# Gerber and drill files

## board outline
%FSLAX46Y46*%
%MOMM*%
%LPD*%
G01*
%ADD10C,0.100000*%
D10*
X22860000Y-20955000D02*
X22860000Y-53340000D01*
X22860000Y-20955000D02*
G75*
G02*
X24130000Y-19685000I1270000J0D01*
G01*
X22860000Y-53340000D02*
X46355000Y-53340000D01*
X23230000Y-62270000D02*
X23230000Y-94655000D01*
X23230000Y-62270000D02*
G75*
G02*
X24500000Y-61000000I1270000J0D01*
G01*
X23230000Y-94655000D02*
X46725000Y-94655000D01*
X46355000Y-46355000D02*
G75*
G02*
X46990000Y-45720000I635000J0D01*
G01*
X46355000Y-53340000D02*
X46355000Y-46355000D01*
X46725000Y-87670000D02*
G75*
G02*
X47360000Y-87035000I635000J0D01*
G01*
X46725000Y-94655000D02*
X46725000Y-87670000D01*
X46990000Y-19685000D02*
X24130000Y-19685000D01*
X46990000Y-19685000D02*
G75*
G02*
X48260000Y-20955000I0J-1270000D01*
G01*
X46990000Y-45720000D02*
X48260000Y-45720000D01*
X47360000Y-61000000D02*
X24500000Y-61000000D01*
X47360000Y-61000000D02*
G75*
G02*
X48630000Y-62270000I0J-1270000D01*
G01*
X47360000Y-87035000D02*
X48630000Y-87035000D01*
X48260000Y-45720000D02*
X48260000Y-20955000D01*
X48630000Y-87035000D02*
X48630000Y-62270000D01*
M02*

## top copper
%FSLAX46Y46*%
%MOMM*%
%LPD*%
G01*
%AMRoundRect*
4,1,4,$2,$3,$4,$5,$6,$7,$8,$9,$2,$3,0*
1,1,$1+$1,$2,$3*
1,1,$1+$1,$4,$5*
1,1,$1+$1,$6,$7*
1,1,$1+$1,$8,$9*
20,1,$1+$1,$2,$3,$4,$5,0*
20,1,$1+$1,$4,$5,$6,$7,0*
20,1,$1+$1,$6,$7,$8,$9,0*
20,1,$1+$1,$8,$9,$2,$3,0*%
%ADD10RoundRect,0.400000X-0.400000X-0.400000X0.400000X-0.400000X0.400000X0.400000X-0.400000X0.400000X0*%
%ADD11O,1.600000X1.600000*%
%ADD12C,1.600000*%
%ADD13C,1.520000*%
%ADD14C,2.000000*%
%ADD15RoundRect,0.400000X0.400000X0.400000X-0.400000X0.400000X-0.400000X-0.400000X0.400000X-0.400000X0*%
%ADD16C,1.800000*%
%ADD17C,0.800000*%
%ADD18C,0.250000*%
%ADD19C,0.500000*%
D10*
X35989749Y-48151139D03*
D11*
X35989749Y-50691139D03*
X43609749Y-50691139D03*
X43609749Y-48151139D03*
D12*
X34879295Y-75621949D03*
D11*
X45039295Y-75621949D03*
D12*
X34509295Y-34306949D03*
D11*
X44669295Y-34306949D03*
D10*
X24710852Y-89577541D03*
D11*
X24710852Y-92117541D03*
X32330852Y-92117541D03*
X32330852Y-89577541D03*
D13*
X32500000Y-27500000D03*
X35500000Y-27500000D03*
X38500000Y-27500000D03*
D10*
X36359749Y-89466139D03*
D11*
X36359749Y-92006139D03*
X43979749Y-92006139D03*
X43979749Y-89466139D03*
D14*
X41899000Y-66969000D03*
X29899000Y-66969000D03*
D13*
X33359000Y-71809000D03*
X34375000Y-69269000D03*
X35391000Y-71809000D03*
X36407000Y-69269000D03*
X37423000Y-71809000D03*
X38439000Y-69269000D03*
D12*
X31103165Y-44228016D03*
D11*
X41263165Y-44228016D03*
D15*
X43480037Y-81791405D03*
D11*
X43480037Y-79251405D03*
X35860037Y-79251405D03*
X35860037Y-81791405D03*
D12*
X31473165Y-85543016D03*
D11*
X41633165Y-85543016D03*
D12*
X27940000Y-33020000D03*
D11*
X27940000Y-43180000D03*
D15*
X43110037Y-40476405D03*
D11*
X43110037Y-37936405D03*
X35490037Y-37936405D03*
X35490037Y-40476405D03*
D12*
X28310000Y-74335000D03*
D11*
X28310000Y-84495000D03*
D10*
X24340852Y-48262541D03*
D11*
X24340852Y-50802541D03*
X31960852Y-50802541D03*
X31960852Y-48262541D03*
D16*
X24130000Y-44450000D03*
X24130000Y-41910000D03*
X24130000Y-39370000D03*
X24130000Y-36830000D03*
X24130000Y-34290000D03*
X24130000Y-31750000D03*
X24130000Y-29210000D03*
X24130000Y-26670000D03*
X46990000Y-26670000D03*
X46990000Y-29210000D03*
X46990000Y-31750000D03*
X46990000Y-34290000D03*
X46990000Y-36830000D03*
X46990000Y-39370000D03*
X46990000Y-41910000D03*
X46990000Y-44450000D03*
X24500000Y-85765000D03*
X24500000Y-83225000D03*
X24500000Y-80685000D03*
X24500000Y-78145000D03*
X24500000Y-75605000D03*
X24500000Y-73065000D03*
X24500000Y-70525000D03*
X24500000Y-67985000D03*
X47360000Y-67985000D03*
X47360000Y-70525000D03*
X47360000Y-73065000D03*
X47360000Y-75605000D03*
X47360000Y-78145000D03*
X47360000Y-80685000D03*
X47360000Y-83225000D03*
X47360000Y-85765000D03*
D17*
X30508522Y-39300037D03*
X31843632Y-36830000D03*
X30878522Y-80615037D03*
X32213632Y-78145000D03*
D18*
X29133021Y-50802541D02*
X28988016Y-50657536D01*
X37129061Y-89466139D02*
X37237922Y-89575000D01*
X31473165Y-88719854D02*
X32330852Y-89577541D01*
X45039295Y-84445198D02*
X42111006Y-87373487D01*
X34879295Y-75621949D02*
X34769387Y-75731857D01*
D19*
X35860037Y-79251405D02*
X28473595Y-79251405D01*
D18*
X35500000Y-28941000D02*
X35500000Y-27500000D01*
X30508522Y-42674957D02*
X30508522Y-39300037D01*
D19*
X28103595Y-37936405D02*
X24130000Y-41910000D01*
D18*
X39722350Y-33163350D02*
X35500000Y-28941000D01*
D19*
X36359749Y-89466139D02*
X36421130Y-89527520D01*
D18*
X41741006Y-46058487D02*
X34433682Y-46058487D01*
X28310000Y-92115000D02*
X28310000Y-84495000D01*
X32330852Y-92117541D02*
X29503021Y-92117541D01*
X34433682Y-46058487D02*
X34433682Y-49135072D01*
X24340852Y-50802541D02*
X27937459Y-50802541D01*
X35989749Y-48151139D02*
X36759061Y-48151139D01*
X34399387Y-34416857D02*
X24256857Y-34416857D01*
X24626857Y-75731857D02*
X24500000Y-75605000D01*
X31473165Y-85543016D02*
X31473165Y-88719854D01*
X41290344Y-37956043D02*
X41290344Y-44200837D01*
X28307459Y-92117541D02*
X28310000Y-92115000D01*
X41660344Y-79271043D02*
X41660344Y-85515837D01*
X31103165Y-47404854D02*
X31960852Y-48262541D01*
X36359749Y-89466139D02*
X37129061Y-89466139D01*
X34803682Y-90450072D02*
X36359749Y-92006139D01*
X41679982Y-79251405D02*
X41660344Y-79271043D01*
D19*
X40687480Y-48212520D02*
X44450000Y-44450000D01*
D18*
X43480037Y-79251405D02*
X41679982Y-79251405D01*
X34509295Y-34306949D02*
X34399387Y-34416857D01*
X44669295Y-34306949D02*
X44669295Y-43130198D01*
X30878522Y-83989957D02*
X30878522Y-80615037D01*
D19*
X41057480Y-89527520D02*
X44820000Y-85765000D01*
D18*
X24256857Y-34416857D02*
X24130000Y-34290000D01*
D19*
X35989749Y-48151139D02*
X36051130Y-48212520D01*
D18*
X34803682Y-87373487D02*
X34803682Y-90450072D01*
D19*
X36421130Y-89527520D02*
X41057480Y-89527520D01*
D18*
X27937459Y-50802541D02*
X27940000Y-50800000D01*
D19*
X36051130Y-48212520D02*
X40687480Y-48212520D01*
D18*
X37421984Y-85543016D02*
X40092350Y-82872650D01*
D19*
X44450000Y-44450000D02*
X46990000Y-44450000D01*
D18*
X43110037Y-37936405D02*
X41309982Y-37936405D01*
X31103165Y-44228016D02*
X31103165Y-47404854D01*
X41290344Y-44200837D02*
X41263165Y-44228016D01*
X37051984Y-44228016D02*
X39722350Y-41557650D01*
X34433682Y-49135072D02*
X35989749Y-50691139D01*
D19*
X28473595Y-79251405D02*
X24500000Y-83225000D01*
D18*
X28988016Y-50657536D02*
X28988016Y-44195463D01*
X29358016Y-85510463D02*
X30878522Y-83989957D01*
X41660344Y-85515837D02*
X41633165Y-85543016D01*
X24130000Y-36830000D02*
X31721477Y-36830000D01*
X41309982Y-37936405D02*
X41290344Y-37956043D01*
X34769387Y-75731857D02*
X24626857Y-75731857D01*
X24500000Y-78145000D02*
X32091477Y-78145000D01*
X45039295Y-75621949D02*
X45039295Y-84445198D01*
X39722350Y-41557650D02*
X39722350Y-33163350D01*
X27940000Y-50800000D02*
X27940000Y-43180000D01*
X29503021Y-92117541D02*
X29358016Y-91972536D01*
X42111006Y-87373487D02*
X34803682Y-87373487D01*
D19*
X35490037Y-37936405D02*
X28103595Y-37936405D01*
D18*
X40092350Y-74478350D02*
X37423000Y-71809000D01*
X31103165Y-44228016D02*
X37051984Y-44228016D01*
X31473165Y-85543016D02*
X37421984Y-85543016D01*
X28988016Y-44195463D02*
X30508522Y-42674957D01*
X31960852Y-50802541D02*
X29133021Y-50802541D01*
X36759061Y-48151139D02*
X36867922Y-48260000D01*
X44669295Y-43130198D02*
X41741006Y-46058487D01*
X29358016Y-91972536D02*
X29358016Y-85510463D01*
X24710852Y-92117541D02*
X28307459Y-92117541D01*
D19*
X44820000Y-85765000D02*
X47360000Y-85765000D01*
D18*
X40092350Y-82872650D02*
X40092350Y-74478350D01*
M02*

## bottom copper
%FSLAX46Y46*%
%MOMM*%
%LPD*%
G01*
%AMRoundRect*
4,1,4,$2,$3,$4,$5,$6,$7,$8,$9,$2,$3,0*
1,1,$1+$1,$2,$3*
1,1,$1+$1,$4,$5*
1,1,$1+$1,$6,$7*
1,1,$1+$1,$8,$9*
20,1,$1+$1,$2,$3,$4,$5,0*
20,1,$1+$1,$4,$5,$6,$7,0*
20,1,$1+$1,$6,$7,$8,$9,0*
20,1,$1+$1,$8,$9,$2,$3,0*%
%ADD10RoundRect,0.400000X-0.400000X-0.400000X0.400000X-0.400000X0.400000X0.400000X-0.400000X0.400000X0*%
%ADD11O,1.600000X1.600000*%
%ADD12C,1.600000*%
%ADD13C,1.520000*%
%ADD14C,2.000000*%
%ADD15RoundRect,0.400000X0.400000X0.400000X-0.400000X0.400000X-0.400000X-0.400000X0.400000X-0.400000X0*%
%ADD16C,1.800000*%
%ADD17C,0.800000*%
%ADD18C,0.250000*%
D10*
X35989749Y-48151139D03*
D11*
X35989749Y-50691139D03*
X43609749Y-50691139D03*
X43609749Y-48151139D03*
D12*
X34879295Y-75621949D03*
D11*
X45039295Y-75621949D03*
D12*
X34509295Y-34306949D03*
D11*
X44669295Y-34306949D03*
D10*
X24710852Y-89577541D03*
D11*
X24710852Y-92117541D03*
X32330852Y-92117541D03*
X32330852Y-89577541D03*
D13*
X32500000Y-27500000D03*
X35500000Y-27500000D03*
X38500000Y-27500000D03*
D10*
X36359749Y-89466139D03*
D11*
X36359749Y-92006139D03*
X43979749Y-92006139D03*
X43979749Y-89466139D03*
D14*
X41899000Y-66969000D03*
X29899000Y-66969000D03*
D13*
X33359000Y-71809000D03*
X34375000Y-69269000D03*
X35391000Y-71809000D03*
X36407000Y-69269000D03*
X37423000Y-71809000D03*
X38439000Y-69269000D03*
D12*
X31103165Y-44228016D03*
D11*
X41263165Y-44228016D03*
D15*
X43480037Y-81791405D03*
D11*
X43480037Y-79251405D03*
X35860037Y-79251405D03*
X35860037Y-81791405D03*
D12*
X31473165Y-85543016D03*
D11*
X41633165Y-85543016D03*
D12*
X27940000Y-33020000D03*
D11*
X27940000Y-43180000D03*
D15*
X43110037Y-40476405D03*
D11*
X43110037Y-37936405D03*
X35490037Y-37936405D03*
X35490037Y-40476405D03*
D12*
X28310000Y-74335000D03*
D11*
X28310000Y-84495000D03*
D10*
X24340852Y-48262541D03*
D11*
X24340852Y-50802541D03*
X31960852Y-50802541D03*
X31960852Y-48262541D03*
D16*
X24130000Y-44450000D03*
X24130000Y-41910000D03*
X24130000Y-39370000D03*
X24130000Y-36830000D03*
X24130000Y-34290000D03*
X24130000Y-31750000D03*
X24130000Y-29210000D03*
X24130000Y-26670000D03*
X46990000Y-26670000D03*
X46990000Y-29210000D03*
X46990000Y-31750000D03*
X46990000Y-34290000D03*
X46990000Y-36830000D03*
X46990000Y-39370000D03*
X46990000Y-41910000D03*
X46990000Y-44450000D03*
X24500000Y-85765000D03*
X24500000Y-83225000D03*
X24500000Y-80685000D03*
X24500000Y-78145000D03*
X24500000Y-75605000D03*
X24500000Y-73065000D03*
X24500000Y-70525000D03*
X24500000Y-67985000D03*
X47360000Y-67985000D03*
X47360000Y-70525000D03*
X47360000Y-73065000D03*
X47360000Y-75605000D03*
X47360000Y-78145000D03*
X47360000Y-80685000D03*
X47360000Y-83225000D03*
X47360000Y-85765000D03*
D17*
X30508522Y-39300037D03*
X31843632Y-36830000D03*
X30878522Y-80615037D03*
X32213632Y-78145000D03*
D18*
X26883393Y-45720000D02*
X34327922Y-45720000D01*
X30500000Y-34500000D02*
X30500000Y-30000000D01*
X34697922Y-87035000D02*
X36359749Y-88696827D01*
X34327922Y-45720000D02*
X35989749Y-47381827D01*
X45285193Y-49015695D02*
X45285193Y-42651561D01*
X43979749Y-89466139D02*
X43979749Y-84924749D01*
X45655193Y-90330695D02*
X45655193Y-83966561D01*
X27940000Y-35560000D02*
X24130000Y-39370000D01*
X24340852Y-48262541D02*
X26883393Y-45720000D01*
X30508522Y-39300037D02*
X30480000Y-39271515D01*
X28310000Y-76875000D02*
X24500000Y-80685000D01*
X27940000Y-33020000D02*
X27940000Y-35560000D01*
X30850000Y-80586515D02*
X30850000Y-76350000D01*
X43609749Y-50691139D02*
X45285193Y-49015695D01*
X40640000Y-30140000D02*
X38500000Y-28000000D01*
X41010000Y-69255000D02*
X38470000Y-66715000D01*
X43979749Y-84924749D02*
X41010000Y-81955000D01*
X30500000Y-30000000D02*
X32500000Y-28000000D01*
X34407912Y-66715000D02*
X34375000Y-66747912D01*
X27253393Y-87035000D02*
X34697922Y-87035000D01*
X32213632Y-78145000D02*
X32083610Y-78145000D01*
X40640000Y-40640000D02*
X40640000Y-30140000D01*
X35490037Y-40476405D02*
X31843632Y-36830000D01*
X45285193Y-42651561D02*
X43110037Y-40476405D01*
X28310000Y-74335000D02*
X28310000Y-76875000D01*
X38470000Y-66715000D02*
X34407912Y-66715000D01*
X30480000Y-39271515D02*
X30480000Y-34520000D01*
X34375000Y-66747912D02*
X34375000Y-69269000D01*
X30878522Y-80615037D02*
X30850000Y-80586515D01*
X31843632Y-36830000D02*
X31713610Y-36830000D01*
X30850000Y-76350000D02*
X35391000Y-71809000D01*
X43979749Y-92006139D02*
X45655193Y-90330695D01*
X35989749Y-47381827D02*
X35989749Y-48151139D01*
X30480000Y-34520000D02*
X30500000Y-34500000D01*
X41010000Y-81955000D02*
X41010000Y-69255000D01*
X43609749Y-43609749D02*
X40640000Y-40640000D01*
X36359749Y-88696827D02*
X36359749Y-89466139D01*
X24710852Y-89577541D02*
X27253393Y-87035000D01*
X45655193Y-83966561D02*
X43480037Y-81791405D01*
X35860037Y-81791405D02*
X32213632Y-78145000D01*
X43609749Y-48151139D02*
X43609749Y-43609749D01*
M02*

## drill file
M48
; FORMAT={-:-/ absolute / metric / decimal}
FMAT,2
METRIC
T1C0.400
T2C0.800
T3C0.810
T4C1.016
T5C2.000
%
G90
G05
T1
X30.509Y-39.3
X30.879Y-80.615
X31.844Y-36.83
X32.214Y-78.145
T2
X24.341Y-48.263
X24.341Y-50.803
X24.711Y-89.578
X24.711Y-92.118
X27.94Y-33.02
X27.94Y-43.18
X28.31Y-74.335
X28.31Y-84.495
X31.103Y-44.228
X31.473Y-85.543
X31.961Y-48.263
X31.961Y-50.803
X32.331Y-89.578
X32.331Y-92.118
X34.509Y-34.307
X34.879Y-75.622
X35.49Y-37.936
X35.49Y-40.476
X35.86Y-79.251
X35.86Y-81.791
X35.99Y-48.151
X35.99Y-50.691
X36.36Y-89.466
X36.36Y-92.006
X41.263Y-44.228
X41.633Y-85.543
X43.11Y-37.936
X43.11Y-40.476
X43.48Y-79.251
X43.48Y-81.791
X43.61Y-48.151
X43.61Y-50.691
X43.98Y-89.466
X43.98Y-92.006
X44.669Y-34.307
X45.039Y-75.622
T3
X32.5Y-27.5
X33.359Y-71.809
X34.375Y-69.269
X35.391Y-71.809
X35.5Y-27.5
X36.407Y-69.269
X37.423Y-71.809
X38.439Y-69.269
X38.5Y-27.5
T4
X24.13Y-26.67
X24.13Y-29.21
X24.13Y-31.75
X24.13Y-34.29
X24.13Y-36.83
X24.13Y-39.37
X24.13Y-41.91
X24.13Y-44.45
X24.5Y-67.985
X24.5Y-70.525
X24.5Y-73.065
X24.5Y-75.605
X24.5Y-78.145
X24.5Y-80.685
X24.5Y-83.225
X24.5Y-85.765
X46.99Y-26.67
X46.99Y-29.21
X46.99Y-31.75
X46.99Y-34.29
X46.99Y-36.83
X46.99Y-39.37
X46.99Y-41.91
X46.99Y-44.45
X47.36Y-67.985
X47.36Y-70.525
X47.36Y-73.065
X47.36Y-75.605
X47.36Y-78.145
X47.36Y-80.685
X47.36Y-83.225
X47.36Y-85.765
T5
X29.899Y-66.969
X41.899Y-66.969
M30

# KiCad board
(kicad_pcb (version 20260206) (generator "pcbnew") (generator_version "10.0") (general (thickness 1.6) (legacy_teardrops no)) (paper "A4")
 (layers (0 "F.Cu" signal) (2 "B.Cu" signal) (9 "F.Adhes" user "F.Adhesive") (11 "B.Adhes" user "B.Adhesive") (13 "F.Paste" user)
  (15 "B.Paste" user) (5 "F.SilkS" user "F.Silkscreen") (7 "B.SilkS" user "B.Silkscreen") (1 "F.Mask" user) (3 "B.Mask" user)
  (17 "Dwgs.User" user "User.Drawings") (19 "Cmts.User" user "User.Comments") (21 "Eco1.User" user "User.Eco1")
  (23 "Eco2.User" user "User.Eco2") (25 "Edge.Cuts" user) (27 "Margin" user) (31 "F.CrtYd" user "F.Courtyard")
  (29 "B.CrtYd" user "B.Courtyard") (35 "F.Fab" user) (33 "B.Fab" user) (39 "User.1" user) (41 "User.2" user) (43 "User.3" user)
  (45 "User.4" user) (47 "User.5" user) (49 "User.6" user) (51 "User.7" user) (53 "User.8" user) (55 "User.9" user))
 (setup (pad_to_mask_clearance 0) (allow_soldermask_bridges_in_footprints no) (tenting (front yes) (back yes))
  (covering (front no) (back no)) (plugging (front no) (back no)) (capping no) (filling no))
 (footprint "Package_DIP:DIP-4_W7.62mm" (layer "F.Cu") (at 35.989749 48.151139)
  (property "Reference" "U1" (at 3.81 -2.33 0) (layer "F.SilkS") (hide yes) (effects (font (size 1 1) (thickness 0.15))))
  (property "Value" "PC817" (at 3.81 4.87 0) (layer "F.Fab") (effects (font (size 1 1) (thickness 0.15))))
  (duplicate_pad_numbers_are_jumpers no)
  (pad "1" thru_hole roundrect (at 0 0) (size 1.6 1.6) (drill 0.8) (layers "*.Cu" "*.Mask") (remove_unused_layers no)
   (roundrect_rratio 0.25))
  (pad "2" thru_hole oval (at 0 2.54) (size 1.6 1.6) (drill 0.8) (layers "*.Cu" "*.Mask") (remove_unused_layers no))
  (pad "3" thru_hole oval (at 7.62 2.54) (size 1.6 1.6) (drill 0.8) (layers "*.Cu" "*.Mask") (remove_unused_layers no))
  (pad "4" thru_hole oval (at 7.62 0) (size 1.6 1.6) (drill 0.8) (layers "*.Cu" "*.Mask") (remove_unused_layers no)))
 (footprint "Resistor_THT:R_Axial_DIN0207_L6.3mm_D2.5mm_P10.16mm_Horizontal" (layer "F.Cu") (at 34.879295 75.621949)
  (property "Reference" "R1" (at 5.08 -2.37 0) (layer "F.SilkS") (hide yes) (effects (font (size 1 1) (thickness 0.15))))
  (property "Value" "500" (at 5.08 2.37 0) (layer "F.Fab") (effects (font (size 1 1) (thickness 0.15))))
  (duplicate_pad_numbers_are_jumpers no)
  (pad "1" thru_hole circle (at 0 0) (size 1.6 1.6) (drill 0.8) (layers "*.Cu" "*.Mask") (remove_unused_layers no))
  (pad "2" thru_hole oval (at 10.16 0) (size 1.6 1.6) (drill 0.8) (layers "*.Cu" "*.Mask") (remove_unused_layers no)))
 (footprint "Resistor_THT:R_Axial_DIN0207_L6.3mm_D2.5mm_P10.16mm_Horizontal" (layer "F.Cu") (at 34.509295 34.306949)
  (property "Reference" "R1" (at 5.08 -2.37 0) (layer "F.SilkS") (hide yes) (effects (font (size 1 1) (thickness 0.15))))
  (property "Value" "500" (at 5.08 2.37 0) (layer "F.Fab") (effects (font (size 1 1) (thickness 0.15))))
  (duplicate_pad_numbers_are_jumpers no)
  (pad "1" thru_hole circle (at 0 0) (size 1.6 1.6) (drill 0.8) (layers "*.Cu" "*.Mask") (remove_unused_layers no))
  (pad "2" thru_hole oval (at 10.16 0) (size 1.6 1.6) (drill 0.8) (layers "*.Cu" "*.Mask") (remove_unused_layers no)))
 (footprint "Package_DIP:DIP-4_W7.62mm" (layer "F.Cu") (at 24.710852 89.577541)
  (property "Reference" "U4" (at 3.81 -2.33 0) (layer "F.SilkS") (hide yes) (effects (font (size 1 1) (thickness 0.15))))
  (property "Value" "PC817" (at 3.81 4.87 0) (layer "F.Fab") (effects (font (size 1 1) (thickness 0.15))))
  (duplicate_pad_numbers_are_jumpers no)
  (pad "1" thru_hole roundrect (at 0 0) (size 1.6 1.6) (drill 0.8) (layers "*.Cu" "*.Mask") (remove_unused_layers no)
   (roundrect_rratio 0.25))
  (pad "2" thru_hole oval (at 0 2.54) (size 1.6 1.6) (drill 0.8) (layers "*.Cu" "*.Mask") (remove_unused_layers no))
  (pad "3" thru_hole oval (at 7.62 2.54) (size 1.6 1.6) (drill 0.8) (layers "*.Cu" "*.Mask") (remove_unused_layers no))
  (pad "4" thru_hole oval (at 7.62 0) (size 1.6 1.6) (drill 0.8) (layers "*.Cu" "*.Mask") (remove_unused_layers no)))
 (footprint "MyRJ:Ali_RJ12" (layer "F.Cu") (at 34.5 25.5 180)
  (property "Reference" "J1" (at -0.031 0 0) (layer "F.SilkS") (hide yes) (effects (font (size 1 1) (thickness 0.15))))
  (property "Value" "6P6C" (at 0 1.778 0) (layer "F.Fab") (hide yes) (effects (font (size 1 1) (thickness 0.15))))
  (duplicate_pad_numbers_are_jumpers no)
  (pad "1" thru_hole circle (at 2 -2) (size 1.52 1.52) (drill 0.81) (layers "*.Cu" "*.Mask") (remove_unused_layers no))
  (pad "2" thru_hole circle (at -1 -2) (size 1.52 1.52) (drill 0.81) (layers "*.Cu" "*.Mask") (remove_unused_layers no))
  (pad "3" thru_hole circle (at -4 -2) (size 1.52 1.52) (drill 0.81) (layers "*.Cu" "*.Mask") (remove_unused_layers no)))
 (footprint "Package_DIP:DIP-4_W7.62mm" (layer "F.Cu") (at 36.359749 89.466139)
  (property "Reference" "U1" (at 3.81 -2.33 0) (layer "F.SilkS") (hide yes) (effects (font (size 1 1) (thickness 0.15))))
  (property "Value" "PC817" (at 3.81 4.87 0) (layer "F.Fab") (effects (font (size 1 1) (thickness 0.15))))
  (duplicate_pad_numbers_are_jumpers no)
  (pad "1" thru_hole roundrect (at 0 0) (size 1.6 1.6) (drill 0.8) (layers "*.Cu" "*.Mask") (remove_unused_layers no)
   (roundrect_rratio 0.25))
  (pad "2" thru_hole oval (at 0 2.54) (size 1.6 1.6) (drill 0.8) (layers "*.Cu" "*.Mask") (remove_unused_layers no))
  (pad "3" thru_hole oval (at 7.62 2.54) (size 1.6 1.6) (drill 0.8) (layers "*.Cu" "*.Mask") (remove_unused_layers no))
  (pad "4" thru_hole oval (at 7.62 0) (size 1.6 1.6) (drill 0.8) (layers "*.Cu" "*.Mask") (remove_unused_layers no)))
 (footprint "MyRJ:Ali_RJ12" (layer "F.Cu") (at 35.899 66.969 180)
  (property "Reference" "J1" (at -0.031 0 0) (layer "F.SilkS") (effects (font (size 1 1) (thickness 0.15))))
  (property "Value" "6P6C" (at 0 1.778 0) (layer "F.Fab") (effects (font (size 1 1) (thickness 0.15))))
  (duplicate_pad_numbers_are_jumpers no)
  (pad "" thru_hole circle (at -6 0 180) (size 2 2) (drill 2) (layers "*.Cu" "*.Mask") (remove_unused_layers no))
  (pad "" thru_hole circle (at 6 0 180) (size 2 2) (drill 2) (layers "*.Cu" "*.Mask") (remove_unused_layers no))
  (pad "1" thru_hole circle (at 2.54 -4.84) (size 1.52 1.52) (drill 0.81) (layers "*.Cu" "*.Mask") (remove_unused_layers no))
  (pad "2" thru_hole circle (at 1.524 -2.3) (size 1.52 1.52) (drill 0.81) (layers "*.Cu" "*.Mask") (remove_unused_layers no))
  (pad "3" thru_hole circle (at 0.508 -4.84) (size 1.52 1.52) (drill 0.81) (layers "*.Cu" "*.Mask") (remove_unused_layers no))
  (pad "4" thru_hole circle (at -0.508 -2.3) (size 1.52 1.52) (drill 0.81) (layers "*.Cu" "*.Mask") (remove_unused_layers no))
  (pad "5" thru_hole circle (at -1.524 -4.84) (size 1.52 1.52) (drill 0.81) (layers "*.Cu" "*.Mask") (remove_unused_layers no))
  (pad "6" thru_hole circle (at -2.54 -2.3) (size 1.52 1.52) (drill 0.81) (layers "*.Cu" "*.Mask") (remove_unused_layers no)))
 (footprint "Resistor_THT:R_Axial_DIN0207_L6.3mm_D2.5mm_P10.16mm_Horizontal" (layer "F.Cu") (at 31.103165 44.228016)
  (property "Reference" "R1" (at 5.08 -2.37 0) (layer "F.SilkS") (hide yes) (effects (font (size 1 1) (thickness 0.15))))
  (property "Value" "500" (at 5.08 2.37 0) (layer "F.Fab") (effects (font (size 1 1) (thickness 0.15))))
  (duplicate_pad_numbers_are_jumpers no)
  (pad "1" thru_hole circle (at 0 0) (size 1.6 1.6) (drill 0.8) (layers "*.Cu" "*.Mask") (remove_unused_layers no))
  (pad "2" thru_hole oval (at 10.16 0) (size 1.6 1.6) (drill 0.8) (layers "*.Cu" "*.Mask") (remove_unused_layers no)))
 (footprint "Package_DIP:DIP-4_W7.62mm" (layer "F.Cu") (at 43.480037 81.791405 180)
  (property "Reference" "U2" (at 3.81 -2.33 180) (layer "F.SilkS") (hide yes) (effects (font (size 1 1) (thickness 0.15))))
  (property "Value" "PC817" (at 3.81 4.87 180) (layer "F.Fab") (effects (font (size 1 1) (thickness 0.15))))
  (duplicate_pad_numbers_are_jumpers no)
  (pad "1" thru_hole roundrect (at 0 0 180) (size 1.6 1.6) (drill 0.8) (layers "*.Cu" "*.Mask") (remove_unused_layers no)
   (roundrect_rratio 0.25))
  (pad "2" thru_hole oval (at 0 2.54 180) (size 1.6 1.6) (drill 0.8) (layers "*.Cu" "*.Mask") (remove_unused_layers no))
  (pad "3" thru_hole oval (at 7.62 2.54 180) (size 1.6 1.6) (drill 0.8) (layers "*.Cu" "*.Mask") (remove_unused_layers no))
  (pad "4" thru_hole oval (at 7.62 0 180) (size 1.6 1.6) (drill 0.8) (layers "*.Cu" "*.Mask") (remove_unused_layers no)))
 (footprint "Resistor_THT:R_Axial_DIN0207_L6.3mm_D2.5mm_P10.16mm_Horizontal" (layer "F.Cu") (at 31.473165 85.543016)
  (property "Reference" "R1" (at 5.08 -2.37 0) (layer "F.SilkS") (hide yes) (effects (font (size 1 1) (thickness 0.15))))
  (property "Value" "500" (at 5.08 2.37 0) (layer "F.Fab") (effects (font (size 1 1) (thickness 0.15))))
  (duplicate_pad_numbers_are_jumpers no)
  (pad "1" thru_hole circle (at 0 0) (size 1.6 1.6) (drill 0.8) (layers "*.Cu" "*.Mask") (remove_unused_layers no))
  (pad "2" thru_hole oval (at 10.16 0) (size 1.6 1.6) (drill 0.8) (layers "*.Cu" "*.Mask") (remove_unused_layers no)))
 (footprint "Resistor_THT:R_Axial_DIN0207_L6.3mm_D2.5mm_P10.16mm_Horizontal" (layer "F.Cu") (at 27.94 33.02 -90)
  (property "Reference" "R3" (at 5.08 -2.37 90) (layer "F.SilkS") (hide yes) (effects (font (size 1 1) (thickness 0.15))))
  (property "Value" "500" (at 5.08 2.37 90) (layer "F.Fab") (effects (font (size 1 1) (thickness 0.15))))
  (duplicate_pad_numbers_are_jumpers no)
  (pad "1" thru_hole circle (at 0 0 270) (size 1.6 1.6) (drill 0.8) (layers "*.Cu" "*.Mask") (remove_unused_layers no))
  (pad "2" thru_hole oval (at 10.16 0 270) (size 1.6 1.6) (drill 0.8) (layers "*.Cu" "*.Mask") (remove_unused_layers no)))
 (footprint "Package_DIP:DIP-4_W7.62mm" (layer "F.Cu") (at 43.110037 40.476405 180)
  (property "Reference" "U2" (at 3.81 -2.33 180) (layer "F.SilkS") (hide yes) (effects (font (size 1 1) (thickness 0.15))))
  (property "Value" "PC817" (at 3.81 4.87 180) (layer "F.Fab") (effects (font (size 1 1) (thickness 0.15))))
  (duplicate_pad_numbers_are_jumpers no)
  (pad "1" thru_hole roundrect (at 0 0 180) (size 1.6 1.6) (drill 0.8) (layers "*.Cu" "*.Mask") (remove_unused_layers no)
   (roundrect_rratio 0.25))
  (pad "2" thru_hole oval (at 0 2.54 180) (size 1.6 1.6) (drill 0.8) (layers "*.Cu" "*.Mask") (remove_unused_layers no))
  (pad "3" thru_hole oval (at 7.62 2.54 180) (size 1.6 1.6) (drill 0.8) (layers "*.Cu" "*.Mask") (remove_unused_layers no))
  (pad "4" thru_hole oval (at 7.62 0 180) (size 1.6 1.6) (drill 0.8) (layers "*.Cu" "*.Mask") (remove_unused_layers no)))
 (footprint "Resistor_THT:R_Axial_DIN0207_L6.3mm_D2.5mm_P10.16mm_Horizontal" (layer "F.Cu") (at 28.31 74.335 -90)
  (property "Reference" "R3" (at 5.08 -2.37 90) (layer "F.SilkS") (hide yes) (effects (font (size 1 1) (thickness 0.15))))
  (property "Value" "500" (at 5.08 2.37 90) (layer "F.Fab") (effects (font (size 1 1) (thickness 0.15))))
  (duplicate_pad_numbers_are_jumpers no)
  (pad "1" thru_hole circle (at 0 0 270) (size 1.6 1.6) (drill 0.8) (layers "*.Cu" "*.Mask") (remove_unused_layers no))
  (pad "2" thru_hole oval (at 10.16 0 270) (size 1.6 1.6) (drill 0.8) (layers "*.Cu" "*.Mask") (remove_unused_layers no)))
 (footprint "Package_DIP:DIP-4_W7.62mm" (layer "F.Cu") (at 24.340852 48.262541)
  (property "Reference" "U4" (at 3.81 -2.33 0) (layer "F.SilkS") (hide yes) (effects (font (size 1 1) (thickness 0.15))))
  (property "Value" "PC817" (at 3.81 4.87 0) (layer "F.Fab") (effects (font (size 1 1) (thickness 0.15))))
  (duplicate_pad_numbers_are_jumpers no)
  (pad "1" thru_hole roundrect (at 0 0) (size 1.6 1.6) (drill 0.8) (layers "*.Cu" "*.Mask") (remove_unused_layers no)
   (roundrect_rratio 0.25))
  (pad "2" thru_hole oval (at 0 2.54) (size 1.6 1.6) (drill 0.8) (layers "*.Cu" "*.Mask") (remove_unused_layers no))
  (pad "3" thru_hole oval (at 7.62 2.54) (size 1.6 1.6) (drill 0.8) (layers "*.Cu" "*.Mask") (remove_unused_layers no))
  (pad "4" thru_hole oval (at 7.62 0) (size 1.6 1.6) (drill 0.8) (layers "*.Cu" "*.Mask") (remove_unused_layers no)))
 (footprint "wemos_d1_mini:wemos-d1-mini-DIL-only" (layer "B.Cu") (at 35.56 35.56 90)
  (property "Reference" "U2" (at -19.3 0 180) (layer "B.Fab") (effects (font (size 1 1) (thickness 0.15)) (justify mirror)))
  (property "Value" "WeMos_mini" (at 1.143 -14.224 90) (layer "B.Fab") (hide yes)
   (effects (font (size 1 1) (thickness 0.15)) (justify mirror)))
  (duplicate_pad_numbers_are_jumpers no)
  (pad "1" thru_hole circle (at -8.89 -11.43 90) (size 1.8 1.8) (drill 1.016) (layers "*.Cu" "*.Mask") (remove_unused_layers no))
  (pad "2" thru_hole circle (at -6.35 -11.43 90) (size 1.8 1.8) (drill 1.016) (layers "*.Cu" "*.Mask") (remove_unused_layers no))
  (pad "3" thru_hole circle (at -3.81 -11.43 90) (size 1.8 1.8) (drill 1.016) (layers "*.Cu" "*.Mask") (remove_unused_layers no))
  (pad "4" thru_hole circle (at -1.27 -11.43 90) (size 1.8 1.8) (drill 1.016) (layers "*.Cu" "*.Mask") (remove_unused_layers no))
  (pad "5" thru_hole circle (at 1.27 -11.43 90) (size 1.8 1.8) (drill 1.016) (layers "*.Cu" "*.Mask") (remove_unused_layers no))
  (pad "6" thru_hole circle (at 3.81 -11.43 90) (size 1.8 1.8) (drill 1.016) (layers "*.Cu" "*.Mask") (remove_unused_layers no))
  (pad "7" thru_hole circle (at 6.35 -11.43 90) (size 1.8 1.8) (drill 1.016) (layers "*.Cu" "*.Mask") (remove_unused_layers no))
  (pad "8" thru_hole circle (at 8.89 -11.43 90) (size 1.8 1.8) (drill 1.016) (layers "*.Cu" "*.Mask") (remove_unused_layers no))
  (pad "9" thru_hole circle (at 8.89 11.43 90) (size 1.8 1.8) (drill 1.016) (layers "*.Cu" "*.Mask") (remove_unused_layers no))
  (pad "10" thru_hole circle (at 6.35 11.43 90) (size 1.8 1.8) (drill 1.016) (layers "*.Cu" "*.Mask") (remove_unused_layers no))
  (pad "11" thru_hole circle (at 3.81 11.43 90) (size 1.8 1.8) (drill 1.016) (layers "*.Cu" "*.Mask") (remove_unused_layers no))
  (pad "12" thru_hole circle (at 1.27 11.43 90) (size 1.8 1.8) (drill 1.016) (layers "*.Cu" "*.Mask") (remove_unused_layers no))
  (pad "13" thru_hole circle (at -1.27 11.43 90) (size 1.8 1.8) (drill 1.016) (layers "*.Cu" "*.Mask") (remove_unused_layers no))
  (pad "14" thru_hole circle (at -3.81 11.43 90) (size 1.8 1.8) (drill 1.016) (layers "*.Cu" "*.Mask") (remove_unused_layers no))
  (pad "15" thru_hole circle (at -6.35 11.43 90) (size 1.8 1.8) (drill 1.016) (layers "*.Cu" "*.Mask") (remove_unused_layers no))
  (pad "16" thru_hole circle (at -8.89 11.43 90) (size 1.8 1.8) (drill 1.016) (layers "*.Cu" "*.Mask") (remove_unused_layers no)))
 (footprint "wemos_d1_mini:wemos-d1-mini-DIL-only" (layer "B.Cu") (at 35.93 76.875 90)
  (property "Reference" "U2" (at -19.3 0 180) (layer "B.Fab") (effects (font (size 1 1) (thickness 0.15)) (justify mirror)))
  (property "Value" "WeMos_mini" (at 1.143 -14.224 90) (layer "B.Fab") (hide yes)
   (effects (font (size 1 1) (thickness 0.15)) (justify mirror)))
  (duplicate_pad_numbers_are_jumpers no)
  (pad "1" thru_hole circle (at -8.89 -11.43 90) (size 1.8 1.8) (drill 1.016) (layers "*.Cu" "*.Mask") (remove_unused_layers no))
  (pad "2" thru_hole circle (at -6.35 -11.43 90) (size 1.8 1.8) (drill 1.016) (layers "*.Cu" "*.Mask") (remove_unused_layers no))
  (pad "3" thru_hole circle (at -3.81 -11.43 90) (size 1.8 1.8) (drill 1.016) (layers "*.Cu" "*.Mask") (remove_unused_layers no))
  (pad "4" thru_hole circle (at -1.27 -11.43 90) (size 1.8 1.8) (drill 1.016) (layers "*.Cu" "*.Mask") (remove_unused_layers no))
  (pad "5" thru_hole circle (at 1.27 -11.43 90) (size 1.8 1.8) (drill 1.016) (layers "*.Cu" "*.Mask") (remove_unused_layers no))
  (pad "6" thru_hole circle (at 3.81 -11.43 90) (size 1.8 1.8) (drill 1.016) (layers "*.Cu" "*.Mask") (remove_unused_layers no))
  (pad "7" thru_hole circle (at 6.35 -11.43 90) (size 1.8 1.8) (drill 1.016) (layers "*.Cu" "*.Mask") (remove_unused_layers no))
  (pad "8" thru_hole circle (at 8.89 -11.43 90) (size 1.8 1.8) (drill 1.016) (layers "*.Cu" "*.Mask") (remove_unused_layers no))
  (pad "9" thru_hole circle (at 8.89 11.43 90) (size 1.8 1.8) (drill 1.016) (layers "*.Cu" "*.Mask") (remove_unused_layers no))
  (pad "10" thru_hole circle (at 6.35 11.43 90) (size 1.8 1.8) (drill 1.016) (layers "*.Cu" "*.Mask") (remove_unused_layers no))
  (pad "11" thru_hole circle (at 3.81 11.43 90) (size 1.8 1.8) (drill 1.016) (layers "*.Cu" "*.Mask") (remove_unused_layers no))
  (pad "12" thru_hole circle (at 1.27 11.43 90) (size 1.8 1.8) (drill 1.016) (layers "*.Cu" "*.Mask") (remove_unused_layers no))
  (pad "13" thru_hole circle (at -1.27 11.43 90) (size 1.8 1.8) (drill 1.016) (layers "*.Cu" "*.Mask") (remove_unused_layers no))
  (pad "14" thru_hole circle (at -3.81 11.43 90) (size 1.8 1.8) (drill 1.016) (layers "*.Cu" "*.Mask") (remove_unused_layers no))
  (pad "15" thru_hole circle (at -6.35 11.43 90) (size 1.8 1.8) (drill 1.016) (layers "*.Cu" "*.Mask") (remove_unused_layers no))
  (pad "16" thru_hole circle (at -8.89 11.43 90) (size 1.8 1.8) (drill 1.016) (layers "*.Cu" "*.Mask") (remove_unused_layers no)))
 (gr_line (start 22.86 20.955) (end 22.86 53.34) (stroke (width 0.1) (type solid)) (layer "Edge.Cuts"))
 (gr_arc (start 22.86 20.955) (mid 23.231974 20.056974) (end 24.13 19.685) (stroke (width 0.1) (type solid)) (layer "Edge.Cuts"))
 (gr_line (start 22.86 53.34) (end 46.355 53.34) (stroke (width 0.1) (type solid)) (layer "Edge.Cuts"))
 (gr_line (start 23.23 62.27) (end 23.23 94.655) (stroke (width 0.1) (type solid)) (layer "Edge.Cuts"))
 (gr_arc (start 23.23 62.27) (mid 23.601974 61.371974) (end 24.5 61) (stroke (width 0.1) (type solid)) (layer "Edge.Cuts"))
 (gr_line (start 23.23 94.655) (end 46.725 94.655) (stroke (width 0.1) (type solid)) (layer "Edge.Cuts"))
 (gr_arc (start 46.355 46.355) (mid 46.540987 45.905987) (end 46.99 45.72) (stroke (width 0.1) (type solid)) (layer "Edge.Cuts"))
 (gr_line (start 46.355 53.34) (end 46.355 46.355) (stroke (width 0.1) (type solid)) (layer "Edge.Cuts"))
 (gr_arc (start 46.725 87.67) (mid 46.910987 87.220987) (end 47.36 87.035) (stroke (width 0.1) (type solid)) (layer "Edge.Cuts"))
 (gr_line (start 46.725 94.655) (end 46.725 87.67) (stroke (width 0.1) (type solid)) (layer "Edge.Cuts"))
 (gr_line (start 46.99 19.685) (end 24.13 19.685) (stroke (width 0.1) (type solid)) (layer "Edge.Cuts"))
 (gr_arc (start 46.99 19.685) (mid 47.888026 20.056974) (end 48.26 20.955) (stroke (width 0.1) (type solid)) (layer "Edge.Cuts"))
 (gr_line (start 46.99 45.72) (end 48.26 45.72) (stroke (width 0.1) (type solid)) (layer "Edge.Cuts"))
 (gr_line (start 47.36 61) (end 24.5 61) (stroke (width 0.1) (type solid)) (layer "Edge.Cuts"))
 (gr_arc (start 47.36 61) (mid 48.258026 61.371974) (end 48.63 62.27) (stroke (width 0.1) (type solid)) (layer "Edge.Cuts"))
 (gr_line (start 47.36 87.035) (end 48.63 87.035) (stroke (width 0.1) (type solid)) (layer "Edge.Cuts"))
 (gr_line (start 48.26 45.72) (end 48.26 20.955) (stroke (width 0.1) (type solid)) (layer "Edge.Cuts"))
 (gr_line (start 48.63 87.035) (end 48.63 62.27) (stroke (width 0.1) (type solid)) (layer "Edge.Cuts"))
 (segment (start 29.133021 50.802541) (end 28.988016 50.657536) (width 0.25) (layer "F.Cu") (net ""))
 (segment (start 37.129061 89.466139) (end 37.237922 89.575) (width 0.25) (layer "F.Cu") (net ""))
 (segment (start 31.473165 88.719854) (end 32.330852 89.577541) (width 0.25) (layer "F.Cu") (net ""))
 (segment (start 45.039295 84.445198) (end 42.111006 87.373487) (width 0.25) (layer "F.Cu") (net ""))
 (segment (start 34.879295 75.621949) (end 34.769387 75.731857) (width 0.25) (layer "F.Cu") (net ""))
 (segment (start 35.860037 79.251405) (end 28.473595 79.251405) (width 0.5) (layer "F.Cu") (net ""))
 (segment (start 35.5 28.941) (end 35.5 27.5) (width 0.25) (layer "F.Cu") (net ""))
 (segment (start 30.508522 42.674957) (end 30.508522 39.300037) (width 0.25) (layer "F.Cu") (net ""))
 (segment (start 28.103595 37.936405) (end 24.13 41.91) (width 0.5) (layer "F.Cu") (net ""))
 (segment (start 39.72235 33.16335) (end 35.5 28.941) (width 0.25) (layer "F.Cu") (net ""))
 (segment (start 36.359749 89.466139) (end 36.42113 89.52752) (width 0.5) (layer "F.Cu") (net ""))
 (segment (start 41.741006 46.058487) (end 34.433682 46.058487) (width 0.25) (layer "F.Cu") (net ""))
 (segment (start 28.31 92.115) (end 28.31 84.495) (width 0.25) (layer "F.Cu") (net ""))
 (segment (start 32.330852 92.117541) (end 29.503021 92.117541) (width 0.25) (layer "F.Cu") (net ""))
 (segment (start 34.433682 46.058487) (end 34.433682 49.135072) (width 0.25) (layer "F.Cu") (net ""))
 (segment (start 24.340852 50.802541) (end 27.937459 50.802541) (width 0.25) (layer "F.Cu") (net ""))
 (segment (start 35.989749 48.151139) (end 36.759061 48.151139) (width 0.25) (layer "F.Cu") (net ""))
 (segment (start 34.399387 34.416857) (end 24.256857 34.416857) (width 0.25) (layer "F.Cu") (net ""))
 (segment (start 24.626857 75.731857) (end 24.5 75.605) (width 0.25) (layer "F.Cu") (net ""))
 (segment (start 31.473165 85.543016) (end 31.473165 88.719854) (width 0.25) (layer "F.Cu") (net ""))
 (segment (start 41.290344 37.956043) (end 41.290344 44.200837) (width 0.25) (layer "F.Cu") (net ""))
 (segment (start 28.307459 92.117541) (end 28.31 92.115) (width 0.25) (layer "F.Cu") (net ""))
 (segment (start 41.660344 79.271043) (end 41.660344 85.515837) (width 0.25) (layer "F.Cu") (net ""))
 (segment (start 31.103165 47.404854) (end 31.960852 48.262541) (width 0.25) (layer "F.Cu") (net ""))
 (segment (start 36.359749 89.466139) (end 37.129061 89.466139) (width 0.25) (layer "F.Cu") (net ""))
 (segment (start 34.803682 90.450072) (end 36.359749 92.006139) (width 0.25) (layer "F.Cu") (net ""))
 (segment (start 41.679982 79.251405) (end 41.660344 79.271043) (width 0.25) (layer "F.Cu") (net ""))
 (segment (start 40.68748 48.21252) (end 44.45 44.45) (width 0.5) (layer "F.Cu") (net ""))
 (segment (start 43.480037 79.251405) (end 41.679982 79.251405) (width 0.25) (layer "F.Cu") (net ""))
 (segment (start 34.509295 34.306949) (end 34.399387 34.416857) (width 0.25) (layer "F.Cu") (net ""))
 (segment (start 44.669295 34.306949) (end 44.669295 43.130198) (width 0.25) (layer "F.Cu") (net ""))
 (segment (start 30.878522 83.989957) (end 30.878522 80.615037) (width 0.25) (layer "F.Cu") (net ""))
 (segment (start 41.05748 89.52752) (end 44.82 85.765) (width 0.5) (layer "F.Cu") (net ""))
 (segment (start 24.256857 34.416857) (end 24.13 34.29) (width 0.25) (layer "F.Cu") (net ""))
 (segment (start 35.989749 48.151139) (end 36.05113 48.21252) (width 0.5) (layer "F.Cu") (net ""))
 (segment (start 34.803682 87.373487) (end 34.803682 90.450072) (width 0.25) (layer "F.Cu") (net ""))
 (segment (start 36.42113 89.52752) (end 41.05748 89.52752) (width 0.5) (layer "F.Cu") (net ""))
 (segment (start 27.937459 50.802541) (end 27.94 50.8) (width 0.25) (layer "F.Cu") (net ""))
 (segment (start 36.05113 48.21252) (end 40.68748 48.21252) (width 0.5) (layer "F.Cu") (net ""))
 (segment (start 37.421984 85.543016) (end 40.09235 82.87265) (width 0.25) (layer "F.Cu") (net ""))
 (segment (start 44.45 44.45) (end 46.99 44.45) (width 0.5) (layer "F.Cu") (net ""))
 (segment (start 43.110037 37.936405) (end 41.309982 37.936405) (width 0.25) (layer "F.Cu") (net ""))
 (segment (start 31.103165 44.228016) (end 31.103165 47.404854) (width 0.25) (layer "F.Cu") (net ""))
 (segment (start 41.290344 44.200837) (end 41.263165 44.228016) (width 0.25) (layer "F.Cu") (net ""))
 (segment (start 37.051984 44.228016) (end 39.72235 41.55765) (width 0.25) (layer "F.Cu") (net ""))
 (segment (start 34.433682 49.135072) (end 35.989749 50.691139) (width 0.25) (layer "F.Cu") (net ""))
 (segment (start 28.473595 79.251405) (end 24.5 83.225) (width 0.5) (layer "F.Cu") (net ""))
 (segment (start 28.988016 50.657536) (end 28.988016 44.195463) (width 0.25) (layer "F.Cu") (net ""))
 (segment (start 29.358016 85.510463) (end 30.878522 83.989957) (width 0.25) (layer "F.Cu") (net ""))
 (segment (start 41.660344 85.515837) (end 41.633165 85.543016) (width 0.25) (layer "F.Cu") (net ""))
 (segment (start 24.13 36.83) (end 31.721477 36.83) (width 0.25) (layer "F.Cu") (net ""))
 (segment (start 41.309982 37.936405) (end 41.290344 37.956043) (width 0.25) (layer "F.Cu") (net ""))
 (segment (start 34.769387 75.731857) (end 24.626857 75.731857) (width 0.25) (layer "F.Cu") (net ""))
 (segment (start 24.5 78.145) (end 32.091477 78.145) (width 0.25) (layer "F.Cu") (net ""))
 (segment (start 45.039295 75.621949) (end 45.039295 84.445198) (width 0.25) (layer "F.Cu") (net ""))
 (segment (start 39.72235 41.55765) (end 39.72235 33.16335) (width 0.25) (layer "F.Cu") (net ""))
 (segment (start 27.94 50.8) (end 27.94 43.18) (width 0.25) (layer "F.Cu") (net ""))
 (segment (start 29.503021 92.117541) (end 29.358016 91.972536) (width 0.25) (layer "F.Cu") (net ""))
 (segment (start 42.111006 87.373487) (end 34.803682 87.373487) (width 0.25) (layer "F.Cu") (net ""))
 (segment (start 35.490037 37.936405) (end 28.103595 37.936405) (width 0.5) (layer "F.Cu") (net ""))
 (segment (start 40.09235 74.47835) (end 37.423 71.809) (width 0.25) (layer "F.Cu") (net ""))
 (segment (start 31.103165 44.228016) (end 37.051984 44.228016) (width 0.25) (layer "F.Cu") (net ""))
 (segment (start 31.473165 85.543016) (end 37.421984 85.543016) (width 0.25) (layer "F.Cu") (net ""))
 (segment (start 28.988016 44.195463) (end 30.508522 42.674957) (width 0.25) (layer "F.Cu") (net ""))
 (segment (start 31.960852 50.802541) (end 29.133021 50.802541) (width 0.25) (layer "F.Cu") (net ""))
 (segment (start 36.759061 48.151139) (end 36.867922 48.26) (width 0.25) (layer "F.Cu") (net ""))
 (segment (start 44.669295 43.130198) (end 41.741006 46.058487) (width 0.25) (layer "F.Cu") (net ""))
 (segment (start 29.358016 91.972536) (end 29.358016 85.510463) (width 0.25) (layer "F.Cu") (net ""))
 (segment (start 24.710852 92.117541) (end 28.307459 92.117541) (width 0.25) (layer "F.Cu") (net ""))
 (segment (start 44.82 85.765) (end 47.36 85.765) (width 0.5) (layer "F.Cu") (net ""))
 (segment (start 40.09235 82.87265) (end 40.09235 74.47835) (width 0.25) (layer "F.Cu") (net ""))
 (via (at 30.508522 39.300037) (size 0.8) (drill 0.4) (layers "F.Cu" "B.Cu") (capping no) (covering (front no) (back no))
  (plugging (front no) (back no)) (filling no) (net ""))
 (via (at 31.843632 36.83) (size 0.8) (drill 0.4) (layers "F.Cu" "B.Cu") (capping no) (covering (front no) (back no))
  (plugging (front no) (back no)) (filling no) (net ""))
 (via (at 30.878522 80.615037) (size 0.8) (drill 0.4) (layers "F.Cu" "B.Cu") (capping no) (covering (front no) (back no))
  (plugging (front no) (back no)) (filling no) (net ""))
 (via (at 32.213632 78.145) (size 0.8) (drill 0.4) (layers "F.Cu" "B.Cu") (capping no) (covering (front no) (back no))
  (plugging (front no) (back no)) (filling no) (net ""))
 (segment (start 26.883393 45.72) (end 34.327922 45.72) (width 0.25) (layer "B.Cu") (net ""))
 (segment (start 30.5 34.5) (end 30.5 30) (width 0.25) (layer "B.Cu") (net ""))
 (segment (start 34.697922 87.035) (end 36.359749 88.696827) (width 0.25) (layer "B.Cu") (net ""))
 (segment (start 34.327922 45.72) (end 35.989749 47.381827) (width 0.25) (layer "B.Cu") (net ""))
 (segment (start 45.285193 49.015695) (end 45.285193 42.651561) (width 0.25) (layer "B.Cu") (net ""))
 (segment (start 43.979749 89.466139) (end 43.979749 84.924749) (width 0.25) (layer "B.Cu") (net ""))
 (segment (start 45.655193 90.330695) (end 45.655193 83.966561) (width 0.25) (layer "B.Cu") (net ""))
 (segment (start 27.94 35.56) (end 24.13 39.37) (width 0.25) (layer "B.Cu") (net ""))
 (segment (start 24.340852 48.262541) (end 26.883393 45.72) (width 0.25) (layer "B.Cu") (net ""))
 (segment (start 30.508522 39.300037) (end 30.48 39.271515) (width 0.25) (layer "B.Cu") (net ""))
 (segment (start 28.31 76.875) (end 24.5 80.685) (width 0.25) (layer "B.Cu") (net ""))
 (segment (start 27.94 33.02) (end 27.94 35.56) (width 0.25) (layer "B.Cu") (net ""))
 (segment (start 30.85 80.586515) (end 30.85 76.35) (width 0.25) (layer "B.Cu") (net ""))
 (segment (start 43.609749 50.691139) (end 45.285193 49.015695) (width 0.25) (layer "B.Cu") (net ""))
 (segment (start 40.64 30.14) (end 38.5 28) (width 0.25) (layer "B.Cu") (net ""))
 (segment (start 41.01 69.255) (end 38.47 66.715) (width 0.25) (layer "B.Cu") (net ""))
 (segment (start 43.979749 84.924749) (end 41.01 81.955) (width 0.25) (layer "B.Cu") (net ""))
 (segment (start 30.5 30) (end 32.5 28) (width 0.25) (layer "B.Cu") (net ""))
 (segment (start 34.407912 66.715) (end 34.375 66.747912) (width 0.25) (layer "B.Cu") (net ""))
 (segment (start 27.253393 87.035) (end 34.697922 87.035) (width 0.25) (layer "B.Cu") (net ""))
 (segment (start 32.213632 78.145) (end 32.08361 78.145) (width 0.25) (layer "B.Cu") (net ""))
 (segment (start 40.64 40.64) (end 40.64 30.14) (width 0.25) (layer "B.Cu") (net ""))
 (segment (start 35.490037 40.476405) (end 31.843632 36.83) (width 0.25) (layer "B.Cu") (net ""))
 (segment (start 45.285193 42.651561) (end 43.110037 40.476405) (width 0.25) (layer "B.Cu") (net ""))
 (segment (start 28.31 74.335) (end 28.31 76.875) (width 0.25) (layer "B.Cu") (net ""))
 (segment (start 38.47 66.715) (end 34.407912 66.715) (width 0.25) (layer "B.Cu") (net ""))
 (segment (start 30.48 39.271515) (end 30.48 34.52) (width 0.25) (layer "B.Cu") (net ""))
 (segment (start 34.375 66.747912) (end 34.375 69.269) (width 0.25) (layer "B.Cu") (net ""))
 (segment (start 30.878522 80.615037) (end 30.85 80.586515) (width 0.25) (layer "B.Cu") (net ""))
 (segment (start 31.843632 36.83) (end 31.71361 36.83) (width 0.25) (layer "B.Cu") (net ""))
 (segment (start 30.85 76.35) (end 35.391 71.809) (width 0.25) (layer "B.Cu") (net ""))
 (segment (start 43.979749 92.006139) (end 45.655193 90.330695) (width 0.25) (layer "B.Cu") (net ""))
 (segment (start 35.989749 47.381827) (end 35.989749 48.151139) (width 0.25) (layer "B.Cu") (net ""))
 (segment (start 30.48 34.52) (end 30.5 34.5) (width 0.25) (layer "B.Cu") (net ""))
 (segment (start 41.01 81.955) (end 41.01 69.255) (width 0.25) (layer "B.Cu") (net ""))
 (segment (start 43.609749 43.609749) (end 40.64 40.64) (width 0.25) (layer "B.Cu") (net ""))
 (segment (start 36.359749 88.696827) (end 36.359749 89.466139) (width 0.25) (layer "B.Cu") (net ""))
 (segment (start 24.710852 89.577541) (end 27.253393 87.035) (width 0.25) (layer "B.Cu") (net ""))
 (segment (start 45.655193 83.966561) (end 43.480037 81.791405) (width 0.25) (layer "B.Cu") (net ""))
 (segment (start 35.860037 81.791405) (end 32.213632 78.145) (width 0.25) (layer "B.Cu") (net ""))
 (segment (start 43.609749 48.151139) (end 43.609749 43.609749) (width 0.25) (layer "B.Cu") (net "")))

